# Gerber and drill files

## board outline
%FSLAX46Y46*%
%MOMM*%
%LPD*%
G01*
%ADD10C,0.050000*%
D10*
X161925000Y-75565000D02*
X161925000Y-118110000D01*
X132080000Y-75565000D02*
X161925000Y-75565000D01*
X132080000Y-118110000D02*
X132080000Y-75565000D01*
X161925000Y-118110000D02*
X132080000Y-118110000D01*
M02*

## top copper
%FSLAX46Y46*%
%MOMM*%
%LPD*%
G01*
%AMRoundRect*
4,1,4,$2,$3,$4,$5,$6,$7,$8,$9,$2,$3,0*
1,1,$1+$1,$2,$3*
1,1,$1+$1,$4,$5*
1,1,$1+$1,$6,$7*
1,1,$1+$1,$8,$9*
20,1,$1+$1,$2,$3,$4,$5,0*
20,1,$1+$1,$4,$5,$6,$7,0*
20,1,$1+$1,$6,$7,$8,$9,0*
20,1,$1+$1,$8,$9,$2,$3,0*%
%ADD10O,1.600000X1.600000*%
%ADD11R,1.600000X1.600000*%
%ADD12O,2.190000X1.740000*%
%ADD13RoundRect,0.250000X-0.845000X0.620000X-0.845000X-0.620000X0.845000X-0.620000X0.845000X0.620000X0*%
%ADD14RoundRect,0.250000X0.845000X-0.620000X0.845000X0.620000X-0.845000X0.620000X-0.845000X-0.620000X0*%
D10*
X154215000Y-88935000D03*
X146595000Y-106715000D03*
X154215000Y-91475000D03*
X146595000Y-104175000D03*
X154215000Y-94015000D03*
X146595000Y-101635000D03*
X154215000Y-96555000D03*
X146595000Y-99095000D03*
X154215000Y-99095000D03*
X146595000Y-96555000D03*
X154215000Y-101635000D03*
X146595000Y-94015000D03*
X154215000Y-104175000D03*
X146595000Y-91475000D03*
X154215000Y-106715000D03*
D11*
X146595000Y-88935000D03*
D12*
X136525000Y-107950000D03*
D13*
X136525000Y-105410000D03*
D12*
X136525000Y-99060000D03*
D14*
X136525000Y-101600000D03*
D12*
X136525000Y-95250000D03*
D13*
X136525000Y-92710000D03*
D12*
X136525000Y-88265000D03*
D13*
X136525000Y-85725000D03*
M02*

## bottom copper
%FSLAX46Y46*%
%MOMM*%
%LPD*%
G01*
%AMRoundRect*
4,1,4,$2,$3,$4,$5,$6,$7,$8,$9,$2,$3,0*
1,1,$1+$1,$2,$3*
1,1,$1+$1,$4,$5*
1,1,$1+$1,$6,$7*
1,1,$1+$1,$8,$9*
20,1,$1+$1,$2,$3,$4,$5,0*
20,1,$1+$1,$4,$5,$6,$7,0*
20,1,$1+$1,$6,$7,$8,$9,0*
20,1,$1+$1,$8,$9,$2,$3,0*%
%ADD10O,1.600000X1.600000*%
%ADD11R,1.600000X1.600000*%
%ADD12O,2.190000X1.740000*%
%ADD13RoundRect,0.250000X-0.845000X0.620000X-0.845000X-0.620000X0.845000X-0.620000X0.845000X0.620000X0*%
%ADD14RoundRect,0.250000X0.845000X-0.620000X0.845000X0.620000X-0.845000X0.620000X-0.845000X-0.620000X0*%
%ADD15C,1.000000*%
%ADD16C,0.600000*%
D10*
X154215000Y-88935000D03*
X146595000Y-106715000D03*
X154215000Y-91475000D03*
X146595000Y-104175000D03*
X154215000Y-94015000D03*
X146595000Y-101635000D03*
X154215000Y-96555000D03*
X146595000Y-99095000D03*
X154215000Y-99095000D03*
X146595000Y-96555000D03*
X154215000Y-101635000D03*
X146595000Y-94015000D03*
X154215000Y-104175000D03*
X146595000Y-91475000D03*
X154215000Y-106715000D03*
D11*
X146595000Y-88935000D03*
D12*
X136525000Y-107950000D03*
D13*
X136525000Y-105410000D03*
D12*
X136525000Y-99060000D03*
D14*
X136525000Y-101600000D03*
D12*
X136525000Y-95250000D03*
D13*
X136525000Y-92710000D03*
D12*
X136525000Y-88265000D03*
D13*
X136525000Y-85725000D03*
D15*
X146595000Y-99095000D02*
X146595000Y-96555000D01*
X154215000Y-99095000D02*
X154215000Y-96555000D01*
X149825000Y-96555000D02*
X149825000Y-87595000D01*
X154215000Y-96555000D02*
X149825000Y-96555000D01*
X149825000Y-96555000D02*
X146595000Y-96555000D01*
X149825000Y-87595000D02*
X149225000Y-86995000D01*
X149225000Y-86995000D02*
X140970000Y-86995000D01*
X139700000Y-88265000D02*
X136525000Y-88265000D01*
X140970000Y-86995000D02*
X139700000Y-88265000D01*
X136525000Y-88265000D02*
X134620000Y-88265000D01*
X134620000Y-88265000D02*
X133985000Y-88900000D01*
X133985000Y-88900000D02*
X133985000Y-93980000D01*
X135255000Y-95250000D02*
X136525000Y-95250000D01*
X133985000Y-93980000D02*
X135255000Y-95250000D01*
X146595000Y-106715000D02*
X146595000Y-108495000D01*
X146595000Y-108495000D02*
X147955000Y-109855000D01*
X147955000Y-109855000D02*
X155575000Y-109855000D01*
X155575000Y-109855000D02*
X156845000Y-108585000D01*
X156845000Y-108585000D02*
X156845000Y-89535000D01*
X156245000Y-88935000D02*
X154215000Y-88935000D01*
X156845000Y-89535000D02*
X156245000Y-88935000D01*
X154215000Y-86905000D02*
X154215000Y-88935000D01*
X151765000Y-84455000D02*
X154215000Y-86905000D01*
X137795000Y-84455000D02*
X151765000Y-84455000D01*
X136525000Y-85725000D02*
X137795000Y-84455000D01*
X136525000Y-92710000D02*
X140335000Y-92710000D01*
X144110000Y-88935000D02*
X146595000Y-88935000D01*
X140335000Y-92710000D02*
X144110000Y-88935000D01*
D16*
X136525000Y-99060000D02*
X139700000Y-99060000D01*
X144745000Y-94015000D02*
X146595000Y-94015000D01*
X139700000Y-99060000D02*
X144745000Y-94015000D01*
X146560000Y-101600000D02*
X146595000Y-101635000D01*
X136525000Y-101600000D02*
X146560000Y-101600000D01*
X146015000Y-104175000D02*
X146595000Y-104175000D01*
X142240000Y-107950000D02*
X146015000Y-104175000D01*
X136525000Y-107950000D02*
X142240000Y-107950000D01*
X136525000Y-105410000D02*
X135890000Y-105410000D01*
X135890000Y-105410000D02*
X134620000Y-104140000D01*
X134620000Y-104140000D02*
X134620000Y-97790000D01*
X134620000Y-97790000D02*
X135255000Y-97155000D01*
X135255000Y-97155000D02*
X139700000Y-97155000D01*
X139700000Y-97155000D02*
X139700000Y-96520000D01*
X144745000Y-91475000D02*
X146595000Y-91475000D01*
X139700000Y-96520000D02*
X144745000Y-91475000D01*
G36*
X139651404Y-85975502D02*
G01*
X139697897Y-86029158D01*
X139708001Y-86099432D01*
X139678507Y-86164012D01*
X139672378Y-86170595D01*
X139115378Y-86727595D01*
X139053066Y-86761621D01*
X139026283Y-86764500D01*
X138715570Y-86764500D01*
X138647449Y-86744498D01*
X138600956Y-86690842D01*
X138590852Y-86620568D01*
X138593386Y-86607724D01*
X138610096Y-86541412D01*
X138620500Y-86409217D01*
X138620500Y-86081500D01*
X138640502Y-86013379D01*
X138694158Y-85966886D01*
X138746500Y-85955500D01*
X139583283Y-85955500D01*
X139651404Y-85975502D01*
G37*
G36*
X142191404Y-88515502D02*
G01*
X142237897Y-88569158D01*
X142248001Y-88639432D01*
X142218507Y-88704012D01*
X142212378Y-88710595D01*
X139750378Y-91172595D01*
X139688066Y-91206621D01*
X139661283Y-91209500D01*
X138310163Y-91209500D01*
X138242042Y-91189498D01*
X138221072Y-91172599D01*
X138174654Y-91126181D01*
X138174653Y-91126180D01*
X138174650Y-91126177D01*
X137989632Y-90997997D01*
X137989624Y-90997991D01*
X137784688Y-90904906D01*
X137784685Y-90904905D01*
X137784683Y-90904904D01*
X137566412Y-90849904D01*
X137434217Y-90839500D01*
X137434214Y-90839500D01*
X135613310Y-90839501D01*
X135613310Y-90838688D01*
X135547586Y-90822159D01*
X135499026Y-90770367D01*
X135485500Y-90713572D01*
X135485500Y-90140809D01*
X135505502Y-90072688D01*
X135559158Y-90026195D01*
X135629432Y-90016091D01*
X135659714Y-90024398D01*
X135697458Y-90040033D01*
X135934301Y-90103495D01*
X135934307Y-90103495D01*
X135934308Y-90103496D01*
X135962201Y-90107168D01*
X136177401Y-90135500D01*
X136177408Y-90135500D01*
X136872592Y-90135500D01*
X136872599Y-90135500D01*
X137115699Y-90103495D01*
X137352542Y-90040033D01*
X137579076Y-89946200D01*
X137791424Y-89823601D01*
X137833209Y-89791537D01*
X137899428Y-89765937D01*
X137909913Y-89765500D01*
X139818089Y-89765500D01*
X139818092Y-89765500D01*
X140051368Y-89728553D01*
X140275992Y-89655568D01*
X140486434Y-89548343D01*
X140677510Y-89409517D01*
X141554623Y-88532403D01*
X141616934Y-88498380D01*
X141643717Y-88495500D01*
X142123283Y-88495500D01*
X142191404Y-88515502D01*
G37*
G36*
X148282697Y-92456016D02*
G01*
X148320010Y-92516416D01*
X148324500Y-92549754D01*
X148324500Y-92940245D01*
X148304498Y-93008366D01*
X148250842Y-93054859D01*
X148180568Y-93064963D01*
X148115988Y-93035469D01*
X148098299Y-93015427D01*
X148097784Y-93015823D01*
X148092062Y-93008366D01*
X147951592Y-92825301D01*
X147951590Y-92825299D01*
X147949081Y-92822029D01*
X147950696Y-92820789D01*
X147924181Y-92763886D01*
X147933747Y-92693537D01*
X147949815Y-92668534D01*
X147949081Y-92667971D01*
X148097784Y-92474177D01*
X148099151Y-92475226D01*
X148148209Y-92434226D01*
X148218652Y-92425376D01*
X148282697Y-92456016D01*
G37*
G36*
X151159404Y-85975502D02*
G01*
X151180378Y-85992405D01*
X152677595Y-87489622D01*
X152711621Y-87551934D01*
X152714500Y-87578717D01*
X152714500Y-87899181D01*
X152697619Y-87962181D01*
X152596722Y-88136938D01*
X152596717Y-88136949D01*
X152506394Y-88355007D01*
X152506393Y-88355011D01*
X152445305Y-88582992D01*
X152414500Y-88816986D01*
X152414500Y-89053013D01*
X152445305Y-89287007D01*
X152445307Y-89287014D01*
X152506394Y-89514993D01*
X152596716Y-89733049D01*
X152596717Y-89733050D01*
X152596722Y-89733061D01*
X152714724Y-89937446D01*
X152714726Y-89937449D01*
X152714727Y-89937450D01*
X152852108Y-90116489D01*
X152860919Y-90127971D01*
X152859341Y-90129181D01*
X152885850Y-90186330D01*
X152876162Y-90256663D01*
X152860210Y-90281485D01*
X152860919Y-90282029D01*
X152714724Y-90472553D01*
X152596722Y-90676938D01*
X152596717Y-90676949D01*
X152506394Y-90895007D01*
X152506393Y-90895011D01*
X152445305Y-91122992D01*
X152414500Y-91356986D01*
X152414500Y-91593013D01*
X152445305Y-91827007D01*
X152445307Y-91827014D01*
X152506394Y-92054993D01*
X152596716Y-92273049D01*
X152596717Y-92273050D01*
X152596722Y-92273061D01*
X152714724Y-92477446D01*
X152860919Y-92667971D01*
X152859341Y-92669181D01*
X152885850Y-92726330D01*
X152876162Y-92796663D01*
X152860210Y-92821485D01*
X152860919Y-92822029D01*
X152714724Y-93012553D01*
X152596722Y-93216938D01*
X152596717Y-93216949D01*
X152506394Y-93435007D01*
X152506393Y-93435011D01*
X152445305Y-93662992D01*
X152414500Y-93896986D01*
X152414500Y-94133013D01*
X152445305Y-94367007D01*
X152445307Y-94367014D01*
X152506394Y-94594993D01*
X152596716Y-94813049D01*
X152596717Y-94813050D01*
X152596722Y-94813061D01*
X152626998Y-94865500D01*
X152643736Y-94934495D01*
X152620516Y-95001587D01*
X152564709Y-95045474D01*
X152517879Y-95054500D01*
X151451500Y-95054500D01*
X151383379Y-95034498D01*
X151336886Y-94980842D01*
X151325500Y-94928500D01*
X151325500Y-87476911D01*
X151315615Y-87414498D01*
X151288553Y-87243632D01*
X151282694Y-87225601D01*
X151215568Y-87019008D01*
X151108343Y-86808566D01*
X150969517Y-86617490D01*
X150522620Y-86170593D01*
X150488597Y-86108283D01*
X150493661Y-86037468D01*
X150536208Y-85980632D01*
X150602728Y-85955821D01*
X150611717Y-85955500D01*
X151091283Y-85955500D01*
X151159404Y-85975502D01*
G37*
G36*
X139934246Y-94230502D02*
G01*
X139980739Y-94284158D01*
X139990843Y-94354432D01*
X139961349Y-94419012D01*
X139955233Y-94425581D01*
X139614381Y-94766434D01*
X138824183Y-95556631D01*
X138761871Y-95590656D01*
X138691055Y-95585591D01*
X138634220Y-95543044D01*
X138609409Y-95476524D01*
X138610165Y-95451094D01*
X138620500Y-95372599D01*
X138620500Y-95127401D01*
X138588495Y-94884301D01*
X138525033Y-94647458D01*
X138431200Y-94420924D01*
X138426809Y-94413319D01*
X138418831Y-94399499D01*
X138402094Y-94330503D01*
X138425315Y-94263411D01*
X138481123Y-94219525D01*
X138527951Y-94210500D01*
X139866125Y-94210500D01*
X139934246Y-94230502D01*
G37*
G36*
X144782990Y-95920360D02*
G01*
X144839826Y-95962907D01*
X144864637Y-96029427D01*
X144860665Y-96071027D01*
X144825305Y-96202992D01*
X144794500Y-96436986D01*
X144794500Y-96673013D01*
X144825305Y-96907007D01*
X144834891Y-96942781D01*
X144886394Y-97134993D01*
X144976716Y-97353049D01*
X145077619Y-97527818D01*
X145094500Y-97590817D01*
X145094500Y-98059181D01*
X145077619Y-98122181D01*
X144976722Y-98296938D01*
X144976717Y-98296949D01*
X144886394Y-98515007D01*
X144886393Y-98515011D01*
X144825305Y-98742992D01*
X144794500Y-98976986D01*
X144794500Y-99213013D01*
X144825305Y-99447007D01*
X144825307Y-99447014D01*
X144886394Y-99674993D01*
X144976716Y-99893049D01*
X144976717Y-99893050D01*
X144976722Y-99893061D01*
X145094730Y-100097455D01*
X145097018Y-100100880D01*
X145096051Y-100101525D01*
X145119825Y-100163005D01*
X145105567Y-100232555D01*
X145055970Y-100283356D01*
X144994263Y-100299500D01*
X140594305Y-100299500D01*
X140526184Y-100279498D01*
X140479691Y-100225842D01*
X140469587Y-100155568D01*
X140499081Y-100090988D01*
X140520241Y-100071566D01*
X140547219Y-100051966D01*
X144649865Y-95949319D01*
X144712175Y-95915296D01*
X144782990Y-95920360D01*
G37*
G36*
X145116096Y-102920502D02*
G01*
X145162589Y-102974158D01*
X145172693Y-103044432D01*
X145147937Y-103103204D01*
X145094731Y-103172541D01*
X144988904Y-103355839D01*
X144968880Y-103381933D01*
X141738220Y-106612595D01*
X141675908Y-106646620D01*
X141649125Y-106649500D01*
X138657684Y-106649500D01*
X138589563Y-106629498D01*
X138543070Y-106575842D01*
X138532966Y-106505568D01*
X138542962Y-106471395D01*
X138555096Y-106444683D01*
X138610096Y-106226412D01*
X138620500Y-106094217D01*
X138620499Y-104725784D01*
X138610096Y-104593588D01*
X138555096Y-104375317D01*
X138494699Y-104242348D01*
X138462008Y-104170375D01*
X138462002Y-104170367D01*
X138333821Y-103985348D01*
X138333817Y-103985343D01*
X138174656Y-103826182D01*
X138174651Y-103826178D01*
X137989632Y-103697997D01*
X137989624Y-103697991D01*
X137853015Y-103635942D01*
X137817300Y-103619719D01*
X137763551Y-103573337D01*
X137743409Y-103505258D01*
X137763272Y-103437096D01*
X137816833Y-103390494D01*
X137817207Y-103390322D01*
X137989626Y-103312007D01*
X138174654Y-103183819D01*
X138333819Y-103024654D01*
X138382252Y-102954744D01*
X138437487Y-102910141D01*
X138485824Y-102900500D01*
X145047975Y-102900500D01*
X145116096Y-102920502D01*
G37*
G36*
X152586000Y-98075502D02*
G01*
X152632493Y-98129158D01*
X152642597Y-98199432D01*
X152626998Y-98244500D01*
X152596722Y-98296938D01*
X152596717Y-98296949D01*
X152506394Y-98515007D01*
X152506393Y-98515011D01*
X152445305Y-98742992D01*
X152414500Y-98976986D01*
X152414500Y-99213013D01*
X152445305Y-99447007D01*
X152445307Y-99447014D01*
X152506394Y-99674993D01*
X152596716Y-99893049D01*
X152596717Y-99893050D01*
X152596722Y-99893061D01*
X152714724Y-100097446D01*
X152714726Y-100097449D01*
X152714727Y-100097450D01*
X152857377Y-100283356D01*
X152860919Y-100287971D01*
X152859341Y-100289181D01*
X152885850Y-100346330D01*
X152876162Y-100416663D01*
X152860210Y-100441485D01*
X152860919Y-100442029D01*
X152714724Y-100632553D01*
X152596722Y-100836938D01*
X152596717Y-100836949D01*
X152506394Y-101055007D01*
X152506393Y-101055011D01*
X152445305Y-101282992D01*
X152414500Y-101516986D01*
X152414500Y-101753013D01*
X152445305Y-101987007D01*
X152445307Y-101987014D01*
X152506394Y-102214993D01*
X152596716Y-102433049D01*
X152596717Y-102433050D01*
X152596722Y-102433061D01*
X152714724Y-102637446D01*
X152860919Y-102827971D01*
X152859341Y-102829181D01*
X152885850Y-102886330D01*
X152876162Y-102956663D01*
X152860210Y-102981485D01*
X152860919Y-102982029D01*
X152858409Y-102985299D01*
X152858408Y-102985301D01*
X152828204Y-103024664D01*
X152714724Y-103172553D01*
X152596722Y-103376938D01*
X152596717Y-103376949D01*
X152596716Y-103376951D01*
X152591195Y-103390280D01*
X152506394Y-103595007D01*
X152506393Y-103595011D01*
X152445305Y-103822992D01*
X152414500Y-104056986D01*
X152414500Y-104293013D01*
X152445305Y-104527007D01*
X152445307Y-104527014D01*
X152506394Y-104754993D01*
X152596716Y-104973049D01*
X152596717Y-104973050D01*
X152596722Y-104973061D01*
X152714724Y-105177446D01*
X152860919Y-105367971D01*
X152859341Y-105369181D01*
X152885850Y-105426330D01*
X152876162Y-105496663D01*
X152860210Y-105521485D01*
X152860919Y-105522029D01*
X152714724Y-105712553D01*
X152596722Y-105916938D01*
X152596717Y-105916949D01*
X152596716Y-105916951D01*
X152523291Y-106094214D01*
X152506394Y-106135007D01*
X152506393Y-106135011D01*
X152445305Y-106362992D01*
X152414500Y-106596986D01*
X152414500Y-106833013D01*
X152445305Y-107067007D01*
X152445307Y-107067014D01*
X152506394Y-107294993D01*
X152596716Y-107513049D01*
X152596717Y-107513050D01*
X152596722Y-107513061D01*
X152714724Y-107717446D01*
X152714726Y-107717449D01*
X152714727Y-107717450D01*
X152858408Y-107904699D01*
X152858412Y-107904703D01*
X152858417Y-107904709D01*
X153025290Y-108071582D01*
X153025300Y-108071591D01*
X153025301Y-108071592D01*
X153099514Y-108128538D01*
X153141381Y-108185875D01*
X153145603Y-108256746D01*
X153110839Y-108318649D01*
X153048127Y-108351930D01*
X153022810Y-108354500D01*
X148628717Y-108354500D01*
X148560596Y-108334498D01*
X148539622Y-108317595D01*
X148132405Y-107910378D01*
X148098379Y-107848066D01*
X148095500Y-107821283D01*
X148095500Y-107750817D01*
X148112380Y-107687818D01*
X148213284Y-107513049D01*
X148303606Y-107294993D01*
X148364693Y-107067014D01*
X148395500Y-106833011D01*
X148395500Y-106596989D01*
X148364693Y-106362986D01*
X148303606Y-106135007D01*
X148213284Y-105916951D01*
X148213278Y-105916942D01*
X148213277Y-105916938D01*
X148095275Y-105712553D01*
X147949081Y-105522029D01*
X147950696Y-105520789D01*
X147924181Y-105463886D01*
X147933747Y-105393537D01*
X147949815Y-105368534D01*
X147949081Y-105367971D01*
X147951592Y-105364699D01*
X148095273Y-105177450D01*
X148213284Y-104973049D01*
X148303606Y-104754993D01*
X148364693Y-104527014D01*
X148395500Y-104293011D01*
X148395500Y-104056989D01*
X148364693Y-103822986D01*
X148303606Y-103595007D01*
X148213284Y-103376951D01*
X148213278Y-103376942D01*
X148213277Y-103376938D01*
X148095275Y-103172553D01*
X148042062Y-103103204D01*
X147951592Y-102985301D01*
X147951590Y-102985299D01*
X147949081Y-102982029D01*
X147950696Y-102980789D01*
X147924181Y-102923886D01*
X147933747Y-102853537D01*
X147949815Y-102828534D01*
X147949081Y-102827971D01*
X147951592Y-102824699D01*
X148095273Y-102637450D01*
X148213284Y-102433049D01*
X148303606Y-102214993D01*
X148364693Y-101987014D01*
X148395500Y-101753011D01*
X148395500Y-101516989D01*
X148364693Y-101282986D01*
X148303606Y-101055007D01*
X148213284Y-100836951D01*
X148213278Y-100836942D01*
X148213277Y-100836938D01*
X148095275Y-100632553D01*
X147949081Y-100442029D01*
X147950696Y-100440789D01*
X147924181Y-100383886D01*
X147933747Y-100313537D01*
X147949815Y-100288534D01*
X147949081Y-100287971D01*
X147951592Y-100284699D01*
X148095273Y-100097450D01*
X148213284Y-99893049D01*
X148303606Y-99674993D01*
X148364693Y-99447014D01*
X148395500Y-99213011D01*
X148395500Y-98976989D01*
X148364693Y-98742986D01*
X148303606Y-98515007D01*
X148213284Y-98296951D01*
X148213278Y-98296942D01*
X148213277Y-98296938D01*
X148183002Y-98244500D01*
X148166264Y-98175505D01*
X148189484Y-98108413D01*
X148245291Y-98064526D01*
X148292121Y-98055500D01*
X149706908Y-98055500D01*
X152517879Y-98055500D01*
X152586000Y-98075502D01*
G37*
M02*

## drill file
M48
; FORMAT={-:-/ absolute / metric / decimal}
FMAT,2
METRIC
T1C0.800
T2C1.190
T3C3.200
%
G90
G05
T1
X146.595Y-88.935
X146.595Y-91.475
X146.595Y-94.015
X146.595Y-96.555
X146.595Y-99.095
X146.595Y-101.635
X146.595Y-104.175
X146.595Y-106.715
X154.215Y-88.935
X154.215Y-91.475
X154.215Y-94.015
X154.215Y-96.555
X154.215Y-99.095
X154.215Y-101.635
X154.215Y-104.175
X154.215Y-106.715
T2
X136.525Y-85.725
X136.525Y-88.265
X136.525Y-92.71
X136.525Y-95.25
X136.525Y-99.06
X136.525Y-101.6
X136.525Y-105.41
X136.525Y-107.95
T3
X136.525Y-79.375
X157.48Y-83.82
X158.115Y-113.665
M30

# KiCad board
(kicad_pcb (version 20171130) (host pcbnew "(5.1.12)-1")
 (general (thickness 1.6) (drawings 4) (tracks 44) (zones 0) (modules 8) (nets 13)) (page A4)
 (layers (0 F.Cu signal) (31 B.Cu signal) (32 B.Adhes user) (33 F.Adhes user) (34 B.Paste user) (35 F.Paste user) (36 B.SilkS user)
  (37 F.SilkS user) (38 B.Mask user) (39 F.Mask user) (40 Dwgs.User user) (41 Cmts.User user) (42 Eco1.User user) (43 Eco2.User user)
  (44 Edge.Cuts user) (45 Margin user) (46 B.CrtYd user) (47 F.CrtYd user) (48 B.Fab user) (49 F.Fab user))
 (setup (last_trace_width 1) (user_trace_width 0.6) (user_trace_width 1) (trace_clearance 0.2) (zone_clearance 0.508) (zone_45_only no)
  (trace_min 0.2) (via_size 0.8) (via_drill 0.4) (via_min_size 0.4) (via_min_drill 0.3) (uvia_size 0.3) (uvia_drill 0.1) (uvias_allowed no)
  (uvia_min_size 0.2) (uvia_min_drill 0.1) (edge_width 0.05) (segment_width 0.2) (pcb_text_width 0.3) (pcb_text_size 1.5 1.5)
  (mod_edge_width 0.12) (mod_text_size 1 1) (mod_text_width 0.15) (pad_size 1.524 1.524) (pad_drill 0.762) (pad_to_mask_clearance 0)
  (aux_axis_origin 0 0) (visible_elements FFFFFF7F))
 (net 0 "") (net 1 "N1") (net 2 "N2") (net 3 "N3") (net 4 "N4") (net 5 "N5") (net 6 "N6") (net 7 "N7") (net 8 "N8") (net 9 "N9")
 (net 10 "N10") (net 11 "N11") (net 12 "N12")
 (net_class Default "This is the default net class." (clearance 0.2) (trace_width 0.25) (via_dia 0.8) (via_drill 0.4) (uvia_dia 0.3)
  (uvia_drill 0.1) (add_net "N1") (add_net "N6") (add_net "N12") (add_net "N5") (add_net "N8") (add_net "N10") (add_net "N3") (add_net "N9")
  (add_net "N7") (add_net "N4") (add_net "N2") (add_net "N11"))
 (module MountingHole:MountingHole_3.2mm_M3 (layer F.Cu) (at 158.115 113.665)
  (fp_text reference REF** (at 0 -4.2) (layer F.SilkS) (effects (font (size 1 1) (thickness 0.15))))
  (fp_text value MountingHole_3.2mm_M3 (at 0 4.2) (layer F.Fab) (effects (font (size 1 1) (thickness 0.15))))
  (pad 1 np_thru_hole circle (at 0 0) (size 3.2 3.2) (drill 3.2) (layers *.Cu *.Mask)))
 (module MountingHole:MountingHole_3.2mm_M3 (layer F.Cu) (at 136.525 79.375)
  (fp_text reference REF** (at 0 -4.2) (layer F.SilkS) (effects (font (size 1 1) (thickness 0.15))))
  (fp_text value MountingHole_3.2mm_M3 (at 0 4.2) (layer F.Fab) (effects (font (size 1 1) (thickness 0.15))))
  (pad 1 np_thru_hole circle (at 0 0) (size 3.2 3.2) (drill 3.2) (layers *.Cu *.Mask)))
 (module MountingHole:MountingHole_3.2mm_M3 (layer F.Cu) (at 157.48 83.82)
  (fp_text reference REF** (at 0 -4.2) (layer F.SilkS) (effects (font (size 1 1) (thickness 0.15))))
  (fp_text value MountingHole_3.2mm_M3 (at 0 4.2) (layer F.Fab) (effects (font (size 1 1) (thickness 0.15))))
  (pad 1 np_thru_hole circle (at 0 0) (size 3.2 3.2) (drill 3.2) (layers *.Cu *.Mask)))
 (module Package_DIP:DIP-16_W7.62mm (layer F.Cu) (at 146.595 88.935)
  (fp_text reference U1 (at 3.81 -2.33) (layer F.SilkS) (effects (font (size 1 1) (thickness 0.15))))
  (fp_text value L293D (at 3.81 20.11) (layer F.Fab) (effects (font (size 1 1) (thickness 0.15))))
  (pad 16 thru_hole oval (at 7.62 0) (size 1.6 1.6) (drill 0.8) (layers *.Cu *.Mask) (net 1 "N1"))
  (pad 8 thru_hole oval (at 0 17.78) (size 1.6 1.6) (drill 0.8) (layers *.Cu *.Mask) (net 1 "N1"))
  (pad 15 thru_hole oval (at 7.62 2.54) (size 1.6 1.6) (drill 0.8) (layers *.Cu *.Mask) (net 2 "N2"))
  (pad 7 thru_hole oval (at 0 15.24) (size 1.6 1.6) (drill 0.8) (layers *.Cu *.Mask) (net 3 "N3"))
  (pad 14 thru_hole oval (at 7.62 5.08) (size 1.6 1.6) (drill 0.8) (layers *.Cu *.Mask) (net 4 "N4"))
  (pad 6 thru_hole oval (at 0 12.7) (size 1.6 1.6) (drill 0.8) (layers *.Cu *.Mask) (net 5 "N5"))
  (pad 13 thru_hole oval (at 7.62 7.62) (size 1.6 1.6) (drill 0.8) (layers *.Cu *.Mask) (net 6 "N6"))
  (pad 5 thru_hole oval (at 0 10.16) (size 1.6 1.6) (drill 0.8) (layers *.Cu *.Mask) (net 6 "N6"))
  (pad 12 thru_hole oval (at 7.62 10.16) (size 1.6 1.6) (drill 0.8) (layers *.Cu *.Mask) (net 6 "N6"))
  (pad 4 thru_hole oval (at 0 7.62) (size 1.6 1.6) (drill 0.8) (layers *.Cu *.Mask) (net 6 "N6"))
  (pad 11 thru_hole oval (at 7.62 12.7) (size 1.6 1.6) (drill 0.8) (layers *.Cu *.Mask) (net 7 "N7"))
  (pad 3 thru_hole oval (at 0 5.08) (size 1.6 1.6) (drill 0.8) (layers *.Cu *.Mask) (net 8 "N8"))
  (pad 10 thru_hole oval (at 7.62 15.24) (size 1.6 1.6) (drill 0.8) (layers *.Cu *.Mask) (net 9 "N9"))
  (pad 2 thru_hole oval (at 0 2.54) (size 1.6 1.6) (drill 0.8) (layers *.Cu *.Mask) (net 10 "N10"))
  (pad 9 thru_hole oval (at 7.62 17.78) (size 1.6 1.6) (drill 0.8) (layers *.Cu *.Mask) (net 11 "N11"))
  (pad 1 thru_hole rect (at 0 0) (size 1.6 1.6) (drill 0.8) (layers *.Cu *.Mask) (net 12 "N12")))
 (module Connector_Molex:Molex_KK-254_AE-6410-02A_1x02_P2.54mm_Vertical (layer F.Cu) (at 136.525 105.41 270)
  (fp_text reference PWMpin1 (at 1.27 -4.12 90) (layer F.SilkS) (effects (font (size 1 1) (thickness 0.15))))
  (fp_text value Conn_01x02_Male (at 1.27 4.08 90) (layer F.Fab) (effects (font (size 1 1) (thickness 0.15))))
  (pad 2 thru_hole oval (at 2.54 0 270) (size 1.74 2.19) (drill 1.19) (layers *.Cu *.Mask) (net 3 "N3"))
  (pad 1 thru_hole roundrect (at 0 0 270) (size 1.74 2.19) (drill 1.19) (layers *.Cu *.Mask) (roundrect_rratio 0.143678) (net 10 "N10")))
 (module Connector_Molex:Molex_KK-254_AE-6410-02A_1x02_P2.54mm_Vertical (layer F.Cu) (at 136.525 101.6 90)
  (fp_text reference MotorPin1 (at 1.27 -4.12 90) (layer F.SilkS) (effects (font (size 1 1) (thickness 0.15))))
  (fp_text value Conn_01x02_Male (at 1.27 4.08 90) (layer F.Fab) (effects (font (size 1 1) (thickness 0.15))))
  (pad 2 thru_hole oval (at 2.54 0 90) (size 1.74 2.19) (drill 1.19) (layers *.Cu *.Mask) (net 8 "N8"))
  (pad 1 thru_hole roundrect (at 0 0 90) (size 1.74 2.19) (drill 1.19) (layers *.Cu *.Mask) (roundrect_rratio 0.143678) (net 5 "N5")))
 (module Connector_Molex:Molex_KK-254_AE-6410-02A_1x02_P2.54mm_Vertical (layer F.Cu) (at 136.525 92.71 270)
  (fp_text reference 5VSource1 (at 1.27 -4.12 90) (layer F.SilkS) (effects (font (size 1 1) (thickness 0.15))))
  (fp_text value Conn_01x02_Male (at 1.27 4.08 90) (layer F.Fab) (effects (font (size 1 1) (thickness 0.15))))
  (pad 2 thru_hole oval (at 2.54 0 270) (size 1.74 2.19) (drill 1.19) (layers *.Cu *.Mask) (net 6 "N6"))
  (pad 1 thru_hole roundrect (at 0 0 270) (size 1.74 2.19) (drill 1.19) (layers *.Cu *.Mask) (roundrect_rratio 0.143678) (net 12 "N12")))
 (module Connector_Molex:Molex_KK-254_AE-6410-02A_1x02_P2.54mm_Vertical (layer F.Cu) (at 136.525 85.725 270)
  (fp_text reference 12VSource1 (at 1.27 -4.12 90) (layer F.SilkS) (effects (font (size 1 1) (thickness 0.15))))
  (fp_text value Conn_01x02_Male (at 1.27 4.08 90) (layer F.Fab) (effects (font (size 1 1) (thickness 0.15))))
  (pad 2 thru_hole oval (at 2.54 0 270) (size 1.74 2.19) (drill 1.19) (layers *.Cu *.Mask) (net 6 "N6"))
  (pad 1 thru_hole roundrect (at 0 0 270) (size 1.74 2.19) (drill 1.19) (layers *.Cu *.Mask) (roundrect_rratio 0.143678) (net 1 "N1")))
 (gr_line (start 161.925 75.565) (end 161.925 118.11) (layer Edge.Cuts) (width 0.05))
 (gr_line (start 132.08 75.565) (end 161.925 75.565) (layer Edge.Cuts) (width 0.05))
 (gr_line (start 132.08 118.11) (end 132.08 75.565) (layer Edge.Cuts) (width 0.05))
 (gr_line (start 161.925 118.11) (end 132.08 118.11) (layer Edge.Cuts) (width 0.05))
 (segment (start 146.595 99.095) (end 146.595 96.555) (width 1) (layer B.Cu) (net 6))
 (segment (start 154.215 99.095) (end 154.215 96.555) (width 1) (layer B.Cu) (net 6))
 (segment (start 149.825 96.555) (end 149.825 87.595) (width 1) (layer B.Cu) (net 6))
 (segment (start 154.215 96.555) (end 149.825 96.555) (width 1) (layer B.Cu) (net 6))
 (segment (start 149.825 96.555) (end 146.595 96.555) (width 1) (layer B.Cu) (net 6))
 (segment (start 149.825 87.595) (end 149.225 86.995) (width 1) (layer B.Cu) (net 6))
 (segment (start 149.225 86.995) (end 140.97 86.995) (width 1) (layer B.Cu) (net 6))
 (segment (start 139.7 88.265) (end 136.525 88.265) (width 1) (layer B.Cu) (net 6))
 (segment (start 140.97 86.995) (end 139.7 88.265) (width 1) (layer B.Cu) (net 6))
 (segment (start 136.525 88.265) (end 134.62 88.265) (width 1) (layer B.Cu) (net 6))
 (segment (start 134.62 88.265) (end 133.985 88.9) (width 1) (layer B.Cu) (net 6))
 (segment (start 133.985 88.9) (end 133.985 93.98) (width 1) (layer B.Cu) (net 6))
 (segment (start 135.255 95.25) (end 136.525 95.25) (width 1) (layer B.Cu) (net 6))
 (segment (start 133.985 93.98) (end 135.255 95.25) (width 1) (layer B.Cu) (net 6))
 (segment (start 146.595 106.715) (end 146.595 108.495) (width 1) (layer B.Cu) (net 1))
 (segment (start 146.595 108.495) (end 147.955 109.855) (width 1) (layer B.Cu) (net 1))
 (segment (start 147.955 109.855) (end 155.575 109.855) (width 1) (layer B.Cu) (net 1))
 (segment (start 155.575 109.855) (end 156.845 108.585) (width 1) (layer B.Cu) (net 1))
 (segment (start 156.845 108.585) (end 156.845 89.535) (width 1) (layer B.Cu) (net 1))
 (segment (start 156.245 88.935) (end 154.215 88.935) (width 1) (layer B.Cu) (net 1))
 (segment (start 156.845 89.535) (end 156.245 88.935) (width 1) (layer B.Cu) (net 1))
 (segment (start 154.215 86.905) (end 154.215 88.935) (width 1) (layer B.Cu) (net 1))
 (segment (start 151.765 84.455) (end 154.215 86.905) (width 1) (layer B.Cu) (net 1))
 (segment (start 137.795 84.455) (end 151.765 84.455) (width 1) (layer B.Cu) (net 1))
 (segment (start 136.525 85.725) (end 137.795 84.455) (width 1) (layer B.Cu) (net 1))
 (segment (start 136.525 92.71) (end 140.335 92.71) (width 1) (layer B.Cu) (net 12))
 (segment (start 144.11 88.935) (end 146.595 88.935) (width 1) (layer B.Cu) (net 12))
 (segment (start 140.335 92.71) (end 144.11 88.935) (width 1) (layer B.Cu) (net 12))
 (segment (start 136.525 99.06) (end 139.7 99.06) (width 0.6) (layer B.Cu) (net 8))
 (segment (start 144.745 94.015) (end 146.595 94.015) (width 0.6) (layer B.Cu) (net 8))
 (segment (start 139.7 99.06) (end 144.745 94.015) (width 0.6) (layer B.Cu) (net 8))
 (segment (start 146.56 101.6) (end 146.595 101.635) (width 0.6) (layer B.Cu) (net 5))
 (segment (start 136.525 101.6) (end 146.56 101.6) (width 0.6) (layer B.Cu) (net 5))
 (segment (start 146.015 104.175) (end 146.595 104.175) (width 0.6) (layer B.Cu) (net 3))
 (segment (start 142.24 107.95) (end 146.015 104.175) (width 0.6) (layer B.Cu) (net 3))
 (segment (start 136.525 107.95) (end 142.24 107.95) (width 0.6) (layer B.Cu) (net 3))
 (segment (start 136.525 105.41) (end 135.89 105.41) (width 0.6) (layer B.Cu) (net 10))
 (segment (start 135.89 105.41) (end 134.62 104.14) (width 0.6) (layer B.Cu) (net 10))
 (segment (start 134.62 104.14) (end 134.62 97.79) (width 0.6) (layer B.Cu) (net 10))
 (segment (start 134.62 97.79) (end 135.255 97.155) (width 0.6) (layer B.Cu) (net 10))
 (segment (start 135.255 97.155) (end 139.7 97.155) (width 0.6) (layer B.Cu) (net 10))
 (segment (start 139.7 97.155) (end 139.7 96.52) (width 0.6) (layer B.Cu) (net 10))
 (segment (start 144.745 91.475) (end 146.595 91.475) (width 0.6) (layer B.Cu) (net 10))
 (segment (start 139.7 96.52) (end 144.745 91.475) (width 0.6) (layer B.Cu) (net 10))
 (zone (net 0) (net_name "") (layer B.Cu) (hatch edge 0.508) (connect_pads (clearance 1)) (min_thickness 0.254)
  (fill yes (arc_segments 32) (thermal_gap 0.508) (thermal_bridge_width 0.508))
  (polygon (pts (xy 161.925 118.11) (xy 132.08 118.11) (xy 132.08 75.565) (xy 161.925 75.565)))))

